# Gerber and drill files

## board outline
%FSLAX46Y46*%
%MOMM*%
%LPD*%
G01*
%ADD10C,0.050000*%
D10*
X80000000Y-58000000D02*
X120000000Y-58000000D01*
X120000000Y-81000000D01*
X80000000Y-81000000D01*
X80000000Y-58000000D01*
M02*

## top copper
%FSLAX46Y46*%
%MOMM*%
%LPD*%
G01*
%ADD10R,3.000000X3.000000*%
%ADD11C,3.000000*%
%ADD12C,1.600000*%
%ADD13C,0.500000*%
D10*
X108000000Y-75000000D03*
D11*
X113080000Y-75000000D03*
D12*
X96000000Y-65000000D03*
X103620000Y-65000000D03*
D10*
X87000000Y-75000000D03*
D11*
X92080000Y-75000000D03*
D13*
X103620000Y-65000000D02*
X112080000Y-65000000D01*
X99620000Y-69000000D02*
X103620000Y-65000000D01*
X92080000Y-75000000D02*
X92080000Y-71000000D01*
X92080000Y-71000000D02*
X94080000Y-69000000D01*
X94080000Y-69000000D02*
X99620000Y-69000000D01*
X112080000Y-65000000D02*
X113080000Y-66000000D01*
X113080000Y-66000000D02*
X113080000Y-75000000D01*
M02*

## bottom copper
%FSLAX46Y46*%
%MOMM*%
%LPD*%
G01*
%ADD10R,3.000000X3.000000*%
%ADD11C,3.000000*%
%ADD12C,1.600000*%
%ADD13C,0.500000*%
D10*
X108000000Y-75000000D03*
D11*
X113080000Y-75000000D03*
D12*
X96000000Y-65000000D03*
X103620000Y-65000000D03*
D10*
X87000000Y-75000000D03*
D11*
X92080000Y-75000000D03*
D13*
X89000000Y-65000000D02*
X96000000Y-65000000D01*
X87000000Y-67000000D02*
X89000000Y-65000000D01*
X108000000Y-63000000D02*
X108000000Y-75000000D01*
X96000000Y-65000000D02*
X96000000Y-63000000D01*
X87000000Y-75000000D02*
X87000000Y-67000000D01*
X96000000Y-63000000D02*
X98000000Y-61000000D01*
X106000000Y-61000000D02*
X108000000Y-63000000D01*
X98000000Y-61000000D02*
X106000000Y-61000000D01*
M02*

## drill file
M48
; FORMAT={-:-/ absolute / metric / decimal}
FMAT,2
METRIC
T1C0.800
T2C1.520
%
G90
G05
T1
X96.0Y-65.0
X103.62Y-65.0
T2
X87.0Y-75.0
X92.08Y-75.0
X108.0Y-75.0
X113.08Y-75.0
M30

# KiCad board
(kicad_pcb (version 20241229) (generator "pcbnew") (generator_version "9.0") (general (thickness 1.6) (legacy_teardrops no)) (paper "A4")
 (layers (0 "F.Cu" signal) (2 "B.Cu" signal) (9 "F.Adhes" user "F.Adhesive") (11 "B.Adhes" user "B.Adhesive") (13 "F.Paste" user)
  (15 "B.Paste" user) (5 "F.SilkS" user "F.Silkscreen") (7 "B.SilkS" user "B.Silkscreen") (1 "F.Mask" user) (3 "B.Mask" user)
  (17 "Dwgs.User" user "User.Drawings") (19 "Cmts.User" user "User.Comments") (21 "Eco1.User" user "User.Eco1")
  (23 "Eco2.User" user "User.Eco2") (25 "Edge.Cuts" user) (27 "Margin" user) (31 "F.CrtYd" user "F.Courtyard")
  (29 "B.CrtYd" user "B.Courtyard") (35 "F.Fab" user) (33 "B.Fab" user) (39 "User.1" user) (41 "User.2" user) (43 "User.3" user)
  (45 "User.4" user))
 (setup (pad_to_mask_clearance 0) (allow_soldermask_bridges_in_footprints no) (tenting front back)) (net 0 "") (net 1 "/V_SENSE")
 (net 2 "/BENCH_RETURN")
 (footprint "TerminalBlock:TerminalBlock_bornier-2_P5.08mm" (layer "F.Cu") (at 108 75)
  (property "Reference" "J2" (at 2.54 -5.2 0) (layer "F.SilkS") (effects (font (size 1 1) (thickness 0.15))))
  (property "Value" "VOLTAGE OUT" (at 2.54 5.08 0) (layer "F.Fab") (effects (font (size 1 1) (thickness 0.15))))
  (pad "1" thru_hole rect (at 0 0) (size 3 3) (drill 1.52) (layers "*.Cu" "*.Mask") (remove_unused_layers no) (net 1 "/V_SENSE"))
  (pad "2" thru_hole circle (at 5.08 0) (size 3 3) (drill 1.52) (layers "*.Cu" "*.Mask") (remove_unused_layers no) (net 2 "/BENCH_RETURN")))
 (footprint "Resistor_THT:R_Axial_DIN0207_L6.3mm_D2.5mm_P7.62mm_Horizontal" (layer "F.Cu") (at 96 65)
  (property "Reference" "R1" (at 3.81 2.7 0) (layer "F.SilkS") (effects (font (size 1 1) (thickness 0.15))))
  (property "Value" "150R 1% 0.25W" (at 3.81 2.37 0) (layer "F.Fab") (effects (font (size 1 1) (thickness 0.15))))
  (pad "1" thru_hole circle (at 0 0) (size 1.6 1.6) (drill 0.8) (layers "*.Cu" "*.Mask") (remove_unused_layers no) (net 1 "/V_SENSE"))
  (pad "2" thru_hole circle (at 7.62 0) (size 1.6 1.6) (drill 0.8) (layers "*.Cu" "*.Mask") (remove_unused_layers no)
   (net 2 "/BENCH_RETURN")))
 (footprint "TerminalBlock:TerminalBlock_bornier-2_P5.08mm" (layer "F.Cu") (at 87 75)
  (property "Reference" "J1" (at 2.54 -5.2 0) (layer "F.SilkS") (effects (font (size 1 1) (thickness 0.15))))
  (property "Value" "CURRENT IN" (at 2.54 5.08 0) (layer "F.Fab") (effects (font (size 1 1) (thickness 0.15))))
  (pad "1" thru_hole rect (at 0 0) (size 3 3) (drill 1.52) (layers "*.Cu" "*.Mask") (remove_unused_layers no) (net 1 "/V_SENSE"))
  (pad "2" thru_hole circle (at 5.08 0) (size 3 3) (drill 1.52) (layers "*.Cu" "*.Mask") (remove_unused_layers no) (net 2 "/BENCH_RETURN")))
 (gr_rect (start 80 58) (end 120 81) (stroke (width 0.05) (type default)) (fill no) (layer "Edge.Cuts"))
 (segment (start 103.62 65) (end 112.08 65) (width 0.5) (layer "F.Cu") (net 2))
 (segment (start 99.62 69) (end 103.62 65) (width 0.5) (layer "F.Cu") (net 2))
 (segment (start 92.08 75) (end 92.08 71) (width 0.5) (layer "F.Cu") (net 2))
 (segment (start 92.08 71) (end 94.08 69) (width 0.5) (layer "F.Cu") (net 2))
 (segment (start 94.08 69) (end 99.62 69) (width 0.5) (layer "F.Cu") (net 2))
 (segment (start 112.08 65) (end 113.08 66) (width 0.5) (layer "F.Cu") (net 2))
 (segment (start 113.08 66) (end 113.08 75) (width 0.5) (layer "F.Cu") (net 2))
 (segment (start 89 65) (end 96 65) (width 0.5) (layer "B.Cu") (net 1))
 (segment (start 87 67) (end 89 65) (width 0.5) (layer "B.Cu") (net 1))
 (segment (start 108 63) (end 108 75) (width 0.5) (layer "B.Cu") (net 1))
 (segment (start 96 65) (end 96 63) (width 0.5) (layer "B.Cu") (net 1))
 (segment (start 87 75) (end 87 67) (width 0.5) (layer "B.Cu") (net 1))
 (segment (start 96 63) (end 98 61) (width 0.5) (layer "B.Cu") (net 1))
 (segment (start 106 61) (end 108 63) (width 0.5) (layer "B.Cu") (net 1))
 (segment (start 98 61) (end 106 61) (width 0.5) (layer "B.Cu") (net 1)))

